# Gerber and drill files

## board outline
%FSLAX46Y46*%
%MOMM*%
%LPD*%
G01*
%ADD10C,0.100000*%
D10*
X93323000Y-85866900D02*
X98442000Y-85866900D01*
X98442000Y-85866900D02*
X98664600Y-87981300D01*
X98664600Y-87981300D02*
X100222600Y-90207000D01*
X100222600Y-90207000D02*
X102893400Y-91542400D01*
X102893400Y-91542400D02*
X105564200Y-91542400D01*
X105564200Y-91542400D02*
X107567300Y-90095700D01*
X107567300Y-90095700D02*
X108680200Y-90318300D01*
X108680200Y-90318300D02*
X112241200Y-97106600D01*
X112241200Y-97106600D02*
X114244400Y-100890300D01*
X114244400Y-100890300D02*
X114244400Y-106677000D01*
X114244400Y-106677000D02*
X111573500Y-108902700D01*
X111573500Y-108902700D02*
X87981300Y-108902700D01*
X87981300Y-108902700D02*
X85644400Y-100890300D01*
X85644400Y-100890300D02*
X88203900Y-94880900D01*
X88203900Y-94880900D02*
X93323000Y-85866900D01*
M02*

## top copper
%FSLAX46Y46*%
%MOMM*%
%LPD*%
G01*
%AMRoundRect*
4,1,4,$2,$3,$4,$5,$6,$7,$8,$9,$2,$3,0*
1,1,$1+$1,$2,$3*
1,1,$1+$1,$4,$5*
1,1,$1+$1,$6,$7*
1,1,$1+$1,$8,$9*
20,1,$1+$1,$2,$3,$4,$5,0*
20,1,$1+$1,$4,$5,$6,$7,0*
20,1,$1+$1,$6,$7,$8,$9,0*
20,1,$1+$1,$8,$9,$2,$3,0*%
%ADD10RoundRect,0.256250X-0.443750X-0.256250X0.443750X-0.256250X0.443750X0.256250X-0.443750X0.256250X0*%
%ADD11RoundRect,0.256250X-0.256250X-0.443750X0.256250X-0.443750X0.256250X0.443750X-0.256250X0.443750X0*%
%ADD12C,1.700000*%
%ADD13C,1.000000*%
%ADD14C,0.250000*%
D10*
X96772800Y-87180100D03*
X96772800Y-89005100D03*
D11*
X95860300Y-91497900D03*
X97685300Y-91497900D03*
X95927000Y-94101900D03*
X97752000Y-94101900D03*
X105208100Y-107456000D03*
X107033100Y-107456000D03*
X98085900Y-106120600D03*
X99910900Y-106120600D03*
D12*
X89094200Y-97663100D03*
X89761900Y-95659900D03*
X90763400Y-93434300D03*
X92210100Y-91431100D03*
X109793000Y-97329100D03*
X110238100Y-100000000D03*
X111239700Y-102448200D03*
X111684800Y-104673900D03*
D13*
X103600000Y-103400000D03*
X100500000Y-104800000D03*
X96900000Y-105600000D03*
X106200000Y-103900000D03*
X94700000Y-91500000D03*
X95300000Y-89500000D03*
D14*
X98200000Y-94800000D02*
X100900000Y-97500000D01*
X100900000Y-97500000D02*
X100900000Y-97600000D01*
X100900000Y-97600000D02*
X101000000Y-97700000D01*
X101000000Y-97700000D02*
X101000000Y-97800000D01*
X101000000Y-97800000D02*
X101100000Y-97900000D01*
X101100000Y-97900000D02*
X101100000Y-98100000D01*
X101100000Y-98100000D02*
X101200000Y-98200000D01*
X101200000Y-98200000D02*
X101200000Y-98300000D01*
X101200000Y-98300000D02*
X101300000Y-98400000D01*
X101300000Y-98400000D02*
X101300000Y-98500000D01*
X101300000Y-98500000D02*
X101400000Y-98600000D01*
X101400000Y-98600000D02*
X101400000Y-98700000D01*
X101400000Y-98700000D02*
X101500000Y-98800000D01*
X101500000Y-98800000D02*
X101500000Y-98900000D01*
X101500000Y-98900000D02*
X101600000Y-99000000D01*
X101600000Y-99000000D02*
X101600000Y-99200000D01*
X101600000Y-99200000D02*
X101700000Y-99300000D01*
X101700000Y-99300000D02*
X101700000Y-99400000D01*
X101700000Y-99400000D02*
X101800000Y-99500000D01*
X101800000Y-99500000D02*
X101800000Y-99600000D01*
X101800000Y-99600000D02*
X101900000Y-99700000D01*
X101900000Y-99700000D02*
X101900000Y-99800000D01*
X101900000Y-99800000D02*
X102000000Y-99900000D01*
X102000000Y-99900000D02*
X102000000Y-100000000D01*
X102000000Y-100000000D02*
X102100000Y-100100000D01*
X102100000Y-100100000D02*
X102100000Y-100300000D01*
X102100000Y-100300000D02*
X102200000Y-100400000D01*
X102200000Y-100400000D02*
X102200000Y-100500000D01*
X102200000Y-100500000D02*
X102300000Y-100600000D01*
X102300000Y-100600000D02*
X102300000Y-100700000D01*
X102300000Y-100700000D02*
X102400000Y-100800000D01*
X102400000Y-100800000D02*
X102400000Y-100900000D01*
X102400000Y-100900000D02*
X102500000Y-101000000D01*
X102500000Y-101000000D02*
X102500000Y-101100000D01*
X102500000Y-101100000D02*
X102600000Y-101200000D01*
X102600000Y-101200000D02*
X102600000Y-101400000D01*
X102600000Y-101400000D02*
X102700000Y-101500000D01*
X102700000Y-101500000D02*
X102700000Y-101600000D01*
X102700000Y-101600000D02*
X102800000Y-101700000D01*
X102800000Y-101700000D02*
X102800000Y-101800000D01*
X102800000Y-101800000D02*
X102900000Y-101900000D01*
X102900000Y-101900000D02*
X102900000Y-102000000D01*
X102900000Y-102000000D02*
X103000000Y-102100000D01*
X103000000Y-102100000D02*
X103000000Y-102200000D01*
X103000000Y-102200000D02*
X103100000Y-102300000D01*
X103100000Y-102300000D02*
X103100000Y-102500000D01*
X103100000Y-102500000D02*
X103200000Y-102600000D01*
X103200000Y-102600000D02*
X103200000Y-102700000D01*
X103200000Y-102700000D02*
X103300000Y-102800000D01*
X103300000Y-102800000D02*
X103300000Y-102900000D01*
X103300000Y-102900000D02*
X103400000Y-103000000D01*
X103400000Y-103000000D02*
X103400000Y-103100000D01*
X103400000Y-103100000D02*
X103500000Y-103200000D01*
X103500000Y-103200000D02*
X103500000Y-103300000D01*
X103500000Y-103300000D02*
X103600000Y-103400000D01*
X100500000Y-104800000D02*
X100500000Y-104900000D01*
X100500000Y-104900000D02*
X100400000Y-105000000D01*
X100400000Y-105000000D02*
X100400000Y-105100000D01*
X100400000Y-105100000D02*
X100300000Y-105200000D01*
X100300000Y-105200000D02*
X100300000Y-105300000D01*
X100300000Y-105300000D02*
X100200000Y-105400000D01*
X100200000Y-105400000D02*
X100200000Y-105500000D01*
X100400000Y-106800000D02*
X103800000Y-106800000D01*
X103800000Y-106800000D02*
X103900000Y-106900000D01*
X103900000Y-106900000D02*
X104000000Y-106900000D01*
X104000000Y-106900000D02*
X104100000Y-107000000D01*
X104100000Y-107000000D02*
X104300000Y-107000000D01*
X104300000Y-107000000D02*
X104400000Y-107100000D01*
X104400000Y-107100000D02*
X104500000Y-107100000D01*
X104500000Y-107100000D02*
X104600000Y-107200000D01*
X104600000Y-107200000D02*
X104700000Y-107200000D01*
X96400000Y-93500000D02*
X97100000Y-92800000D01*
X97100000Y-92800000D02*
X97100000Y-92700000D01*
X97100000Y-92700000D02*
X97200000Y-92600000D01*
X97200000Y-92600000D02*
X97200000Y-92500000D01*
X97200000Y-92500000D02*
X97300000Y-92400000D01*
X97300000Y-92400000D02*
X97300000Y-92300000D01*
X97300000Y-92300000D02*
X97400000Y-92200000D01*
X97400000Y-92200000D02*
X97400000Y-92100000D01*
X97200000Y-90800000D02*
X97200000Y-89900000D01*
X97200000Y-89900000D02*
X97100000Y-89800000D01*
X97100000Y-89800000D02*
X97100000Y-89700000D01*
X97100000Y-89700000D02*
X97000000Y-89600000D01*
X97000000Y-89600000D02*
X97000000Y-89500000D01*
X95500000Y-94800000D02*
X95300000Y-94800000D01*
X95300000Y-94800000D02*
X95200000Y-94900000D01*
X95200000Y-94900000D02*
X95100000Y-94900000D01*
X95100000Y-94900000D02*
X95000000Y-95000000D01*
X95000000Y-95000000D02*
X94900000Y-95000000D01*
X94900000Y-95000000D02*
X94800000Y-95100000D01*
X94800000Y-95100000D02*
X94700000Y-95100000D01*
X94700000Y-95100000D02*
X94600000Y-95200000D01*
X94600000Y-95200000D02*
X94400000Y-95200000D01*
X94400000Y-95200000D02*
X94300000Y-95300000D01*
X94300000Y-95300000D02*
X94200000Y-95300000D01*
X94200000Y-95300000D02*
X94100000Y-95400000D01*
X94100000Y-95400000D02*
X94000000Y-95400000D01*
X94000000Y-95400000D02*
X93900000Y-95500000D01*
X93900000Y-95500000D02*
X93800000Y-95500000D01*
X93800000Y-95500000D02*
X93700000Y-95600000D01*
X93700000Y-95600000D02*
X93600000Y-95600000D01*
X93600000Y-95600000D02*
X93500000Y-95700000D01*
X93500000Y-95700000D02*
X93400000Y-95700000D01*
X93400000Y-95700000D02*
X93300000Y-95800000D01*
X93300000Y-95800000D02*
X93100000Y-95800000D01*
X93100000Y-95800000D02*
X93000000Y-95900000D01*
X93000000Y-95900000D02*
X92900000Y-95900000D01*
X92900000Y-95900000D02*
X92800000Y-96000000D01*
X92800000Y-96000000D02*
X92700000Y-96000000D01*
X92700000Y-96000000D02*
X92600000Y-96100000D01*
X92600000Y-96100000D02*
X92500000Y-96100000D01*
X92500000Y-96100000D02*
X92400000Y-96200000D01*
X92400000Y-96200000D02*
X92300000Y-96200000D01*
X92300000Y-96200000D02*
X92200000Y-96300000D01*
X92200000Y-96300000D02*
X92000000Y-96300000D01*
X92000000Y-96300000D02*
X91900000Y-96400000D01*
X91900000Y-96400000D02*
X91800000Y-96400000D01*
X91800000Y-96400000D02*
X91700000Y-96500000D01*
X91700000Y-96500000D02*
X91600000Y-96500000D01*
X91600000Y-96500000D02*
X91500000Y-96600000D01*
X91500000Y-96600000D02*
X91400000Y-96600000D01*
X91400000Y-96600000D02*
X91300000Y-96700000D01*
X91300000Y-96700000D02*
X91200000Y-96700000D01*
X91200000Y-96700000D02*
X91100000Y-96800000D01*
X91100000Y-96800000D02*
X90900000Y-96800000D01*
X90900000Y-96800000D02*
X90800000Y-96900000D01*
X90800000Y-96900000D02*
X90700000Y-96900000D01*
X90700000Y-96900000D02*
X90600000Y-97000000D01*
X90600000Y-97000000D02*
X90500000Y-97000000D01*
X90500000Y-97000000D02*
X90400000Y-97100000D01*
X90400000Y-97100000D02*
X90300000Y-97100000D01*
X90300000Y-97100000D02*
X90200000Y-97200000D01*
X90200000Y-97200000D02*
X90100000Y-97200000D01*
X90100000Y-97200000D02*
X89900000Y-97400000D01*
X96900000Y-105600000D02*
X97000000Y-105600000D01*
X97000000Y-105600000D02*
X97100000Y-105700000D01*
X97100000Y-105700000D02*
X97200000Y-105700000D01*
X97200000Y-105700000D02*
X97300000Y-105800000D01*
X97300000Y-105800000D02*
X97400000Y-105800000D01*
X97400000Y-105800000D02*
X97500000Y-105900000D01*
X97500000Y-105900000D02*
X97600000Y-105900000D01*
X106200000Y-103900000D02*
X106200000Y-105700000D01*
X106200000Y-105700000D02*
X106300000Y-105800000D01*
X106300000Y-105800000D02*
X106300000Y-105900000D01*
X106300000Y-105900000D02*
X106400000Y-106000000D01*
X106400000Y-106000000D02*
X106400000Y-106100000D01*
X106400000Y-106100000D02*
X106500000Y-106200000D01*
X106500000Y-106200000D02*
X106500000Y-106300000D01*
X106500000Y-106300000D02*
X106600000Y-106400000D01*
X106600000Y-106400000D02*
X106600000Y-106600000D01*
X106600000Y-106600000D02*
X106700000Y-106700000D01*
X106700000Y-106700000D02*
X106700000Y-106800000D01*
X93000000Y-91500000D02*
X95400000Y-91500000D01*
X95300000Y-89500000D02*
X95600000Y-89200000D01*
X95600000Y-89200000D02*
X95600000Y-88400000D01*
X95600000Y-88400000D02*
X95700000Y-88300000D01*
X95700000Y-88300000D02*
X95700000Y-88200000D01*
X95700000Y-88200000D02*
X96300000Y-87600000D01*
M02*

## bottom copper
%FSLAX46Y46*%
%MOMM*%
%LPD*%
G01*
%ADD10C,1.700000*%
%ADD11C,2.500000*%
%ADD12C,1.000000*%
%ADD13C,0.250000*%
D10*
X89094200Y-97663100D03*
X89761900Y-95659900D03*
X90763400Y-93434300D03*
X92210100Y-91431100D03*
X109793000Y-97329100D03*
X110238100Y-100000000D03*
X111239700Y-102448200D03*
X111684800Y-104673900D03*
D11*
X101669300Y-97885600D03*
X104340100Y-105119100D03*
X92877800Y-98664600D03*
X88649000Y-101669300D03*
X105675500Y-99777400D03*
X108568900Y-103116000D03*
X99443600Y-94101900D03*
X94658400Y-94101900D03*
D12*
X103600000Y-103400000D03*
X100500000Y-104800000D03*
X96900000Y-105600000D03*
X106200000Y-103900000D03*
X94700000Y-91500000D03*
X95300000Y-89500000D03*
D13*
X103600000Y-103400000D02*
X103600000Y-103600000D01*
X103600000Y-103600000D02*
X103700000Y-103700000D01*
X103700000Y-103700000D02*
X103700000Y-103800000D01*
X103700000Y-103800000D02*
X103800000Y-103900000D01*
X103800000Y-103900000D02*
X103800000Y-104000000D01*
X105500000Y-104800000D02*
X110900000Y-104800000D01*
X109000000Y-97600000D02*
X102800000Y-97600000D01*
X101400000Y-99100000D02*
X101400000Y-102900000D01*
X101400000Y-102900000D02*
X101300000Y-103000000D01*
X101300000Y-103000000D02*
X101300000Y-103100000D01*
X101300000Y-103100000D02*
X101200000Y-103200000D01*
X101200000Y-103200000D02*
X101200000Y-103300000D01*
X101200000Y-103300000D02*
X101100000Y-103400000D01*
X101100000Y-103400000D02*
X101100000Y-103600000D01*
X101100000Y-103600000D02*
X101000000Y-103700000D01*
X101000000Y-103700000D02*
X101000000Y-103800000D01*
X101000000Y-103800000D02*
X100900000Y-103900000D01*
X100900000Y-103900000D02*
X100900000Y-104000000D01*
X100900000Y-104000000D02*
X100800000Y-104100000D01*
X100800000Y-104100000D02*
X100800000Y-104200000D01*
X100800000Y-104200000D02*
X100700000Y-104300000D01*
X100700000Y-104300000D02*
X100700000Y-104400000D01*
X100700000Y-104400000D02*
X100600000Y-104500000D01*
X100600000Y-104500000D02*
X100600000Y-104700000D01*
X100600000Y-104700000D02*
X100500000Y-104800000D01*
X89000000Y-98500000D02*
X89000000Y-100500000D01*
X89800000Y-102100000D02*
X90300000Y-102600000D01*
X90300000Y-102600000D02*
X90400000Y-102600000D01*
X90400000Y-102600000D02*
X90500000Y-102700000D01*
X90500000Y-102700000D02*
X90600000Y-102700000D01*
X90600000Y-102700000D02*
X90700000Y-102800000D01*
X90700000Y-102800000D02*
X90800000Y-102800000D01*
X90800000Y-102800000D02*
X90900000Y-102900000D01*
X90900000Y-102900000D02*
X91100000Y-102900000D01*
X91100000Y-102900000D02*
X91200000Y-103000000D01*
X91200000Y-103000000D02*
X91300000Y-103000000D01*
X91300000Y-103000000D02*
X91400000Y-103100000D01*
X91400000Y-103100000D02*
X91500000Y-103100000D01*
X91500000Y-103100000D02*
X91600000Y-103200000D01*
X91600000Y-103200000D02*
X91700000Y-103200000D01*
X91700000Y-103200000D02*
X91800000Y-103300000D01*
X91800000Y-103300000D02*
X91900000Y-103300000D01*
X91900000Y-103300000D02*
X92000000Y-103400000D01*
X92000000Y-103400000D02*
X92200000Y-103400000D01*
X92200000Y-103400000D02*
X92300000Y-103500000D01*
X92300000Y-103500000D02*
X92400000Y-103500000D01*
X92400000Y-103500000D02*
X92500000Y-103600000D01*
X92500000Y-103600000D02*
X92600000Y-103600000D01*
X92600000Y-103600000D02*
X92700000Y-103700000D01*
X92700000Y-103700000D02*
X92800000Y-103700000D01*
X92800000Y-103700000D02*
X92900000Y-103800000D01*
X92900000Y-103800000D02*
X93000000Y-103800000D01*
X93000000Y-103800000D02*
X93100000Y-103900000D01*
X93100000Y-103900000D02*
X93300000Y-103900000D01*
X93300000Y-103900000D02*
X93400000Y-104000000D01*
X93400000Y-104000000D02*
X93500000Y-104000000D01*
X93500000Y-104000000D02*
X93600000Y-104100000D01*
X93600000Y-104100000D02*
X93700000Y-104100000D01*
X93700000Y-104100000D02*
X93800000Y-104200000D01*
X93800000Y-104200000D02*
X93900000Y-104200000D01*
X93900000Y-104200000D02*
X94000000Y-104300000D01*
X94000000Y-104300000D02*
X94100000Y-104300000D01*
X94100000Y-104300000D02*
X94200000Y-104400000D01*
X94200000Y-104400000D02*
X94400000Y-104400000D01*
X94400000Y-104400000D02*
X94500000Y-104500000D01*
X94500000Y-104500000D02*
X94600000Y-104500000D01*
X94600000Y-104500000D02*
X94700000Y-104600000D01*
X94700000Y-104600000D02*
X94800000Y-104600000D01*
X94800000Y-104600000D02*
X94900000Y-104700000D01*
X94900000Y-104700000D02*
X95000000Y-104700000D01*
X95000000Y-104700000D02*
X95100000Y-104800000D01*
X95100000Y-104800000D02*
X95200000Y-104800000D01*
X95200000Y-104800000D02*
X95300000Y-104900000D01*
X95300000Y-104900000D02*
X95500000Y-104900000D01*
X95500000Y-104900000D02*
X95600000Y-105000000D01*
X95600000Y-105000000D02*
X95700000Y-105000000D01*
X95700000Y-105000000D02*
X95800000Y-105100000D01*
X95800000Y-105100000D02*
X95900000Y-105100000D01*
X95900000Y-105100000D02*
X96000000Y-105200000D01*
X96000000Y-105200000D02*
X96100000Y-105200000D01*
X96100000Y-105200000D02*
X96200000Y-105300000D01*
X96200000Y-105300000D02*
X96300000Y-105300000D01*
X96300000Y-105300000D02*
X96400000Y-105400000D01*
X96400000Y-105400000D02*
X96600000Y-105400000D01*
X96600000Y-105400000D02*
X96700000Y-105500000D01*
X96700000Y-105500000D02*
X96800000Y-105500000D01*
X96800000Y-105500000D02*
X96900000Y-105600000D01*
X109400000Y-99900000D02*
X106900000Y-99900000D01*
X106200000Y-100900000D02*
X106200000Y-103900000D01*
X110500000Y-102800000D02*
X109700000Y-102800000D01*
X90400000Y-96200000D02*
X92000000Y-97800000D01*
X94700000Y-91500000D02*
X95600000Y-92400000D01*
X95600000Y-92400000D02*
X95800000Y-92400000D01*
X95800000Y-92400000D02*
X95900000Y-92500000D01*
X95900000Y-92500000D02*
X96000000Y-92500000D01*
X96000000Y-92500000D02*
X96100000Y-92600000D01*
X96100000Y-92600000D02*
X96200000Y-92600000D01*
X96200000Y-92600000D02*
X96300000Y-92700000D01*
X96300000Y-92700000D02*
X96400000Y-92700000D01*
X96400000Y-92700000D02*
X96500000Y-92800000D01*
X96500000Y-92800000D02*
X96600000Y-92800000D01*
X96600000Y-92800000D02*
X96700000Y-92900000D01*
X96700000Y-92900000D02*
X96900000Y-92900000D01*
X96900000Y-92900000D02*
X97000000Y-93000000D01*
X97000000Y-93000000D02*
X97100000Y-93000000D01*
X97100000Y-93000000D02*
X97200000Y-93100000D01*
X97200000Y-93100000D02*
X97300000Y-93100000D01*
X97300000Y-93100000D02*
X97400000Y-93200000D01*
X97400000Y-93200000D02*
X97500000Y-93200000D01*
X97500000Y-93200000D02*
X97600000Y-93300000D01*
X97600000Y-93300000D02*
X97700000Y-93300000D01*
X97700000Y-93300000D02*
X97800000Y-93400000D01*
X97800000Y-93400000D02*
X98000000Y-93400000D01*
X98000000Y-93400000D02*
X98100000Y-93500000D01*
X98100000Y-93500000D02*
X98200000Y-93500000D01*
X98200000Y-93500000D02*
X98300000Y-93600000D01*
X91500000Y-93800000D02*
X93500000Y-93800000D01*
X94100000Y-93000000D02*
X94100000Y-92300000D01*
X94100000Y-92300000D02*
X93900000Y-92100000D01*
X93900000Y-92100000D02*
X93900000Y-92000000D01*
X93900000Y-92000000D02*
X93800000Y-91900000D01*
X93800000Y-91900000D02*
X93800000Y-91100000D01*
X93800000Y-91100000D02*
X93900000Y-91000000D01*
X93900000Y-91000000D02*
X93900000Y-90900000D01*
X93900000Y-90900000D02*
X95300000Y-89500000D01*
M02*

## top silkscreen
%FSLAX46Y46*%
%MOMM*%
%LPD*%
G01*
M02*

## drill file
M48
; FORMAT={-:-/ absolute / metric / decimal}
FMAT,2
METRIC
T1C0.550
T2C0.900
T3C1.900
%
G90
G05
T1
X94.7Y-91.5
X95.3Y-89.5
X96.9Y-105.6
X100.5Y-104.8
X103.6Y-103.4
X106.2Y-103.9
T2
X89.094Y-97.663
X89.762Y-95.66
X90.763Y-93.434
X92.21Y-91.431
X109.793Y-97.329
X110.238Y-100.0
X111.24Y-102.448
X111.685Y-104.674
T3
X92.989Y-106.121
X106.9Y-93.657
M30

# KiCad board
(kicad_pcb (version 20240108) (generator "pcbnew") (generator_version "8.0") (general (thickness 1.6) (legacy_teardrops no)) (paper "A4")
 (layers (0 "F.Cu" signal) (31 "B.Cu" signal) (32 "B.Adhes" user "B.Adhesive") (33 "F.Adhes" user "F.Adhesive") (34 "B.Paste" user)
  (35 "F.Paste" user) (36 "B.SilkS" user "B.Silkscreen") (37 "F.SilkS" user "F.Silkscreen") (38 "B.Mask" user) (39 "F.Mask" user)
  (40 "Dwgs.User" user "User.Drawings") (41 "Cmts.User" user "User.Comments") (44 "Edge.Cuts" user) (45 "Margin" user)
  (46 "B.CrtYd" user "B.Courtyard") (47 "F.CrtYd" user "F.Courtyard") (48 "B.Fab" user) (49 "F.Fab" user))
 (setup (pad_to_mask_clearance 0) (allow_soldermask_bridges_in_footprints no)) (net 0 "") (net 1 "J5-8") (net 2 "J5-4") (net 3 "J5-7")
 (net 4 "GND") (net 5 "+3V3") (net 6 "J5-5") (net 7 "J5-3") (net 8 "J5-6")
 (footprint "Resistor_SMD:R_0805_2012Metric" (layer "F.Cu") (at 96.7728 88.0926)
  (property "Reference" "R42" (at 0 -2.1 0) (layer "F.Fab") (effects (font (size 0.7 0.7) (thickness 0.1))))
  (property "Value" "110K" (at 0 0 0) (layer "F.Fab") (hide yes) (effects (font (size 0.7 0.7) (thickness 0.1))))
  (pad "1" smd roundrect (at 0 -0.9125) (size 1.4 1.025) (layers "F.Cu" "F.Mask" "F.Paste") (roundrect_rratio 0.25) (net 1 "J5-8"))
  (pad "2" smd roundrect (at 0 0.9125) (size 1.4 1.025) (layers "F.Cu" "F.Mask" "F.Paste") (roundrect_rratio 0.25) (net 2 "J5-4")))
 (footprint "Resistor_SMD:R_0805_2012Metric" (layer "F.Cu") (at 96.7728 91.4979)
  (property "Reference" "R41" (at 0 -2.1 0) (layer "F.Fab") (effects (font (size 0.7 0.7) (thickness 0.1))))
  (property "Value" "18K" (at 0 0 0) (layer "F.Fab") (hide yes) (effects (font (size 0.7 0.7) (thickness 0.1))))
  (pad "1" smd roundrect (at -0.9125 0) (size 1.025 1.4) (layers "F.Cu" "F.Mask" "F.Paste") (roundrect_rratio 0.25) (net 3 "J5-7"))
  (pad "2" smd roundrect (at 0.9125 0) (size 1.025 1.4) (layers "F.Cu" "F.Mask" "F.Paste") (roundrect_rratio 0.25) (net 2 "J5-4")))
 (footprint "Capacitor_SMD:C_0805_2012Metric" (layer "F.Cu") (at 96.8395 94.1019)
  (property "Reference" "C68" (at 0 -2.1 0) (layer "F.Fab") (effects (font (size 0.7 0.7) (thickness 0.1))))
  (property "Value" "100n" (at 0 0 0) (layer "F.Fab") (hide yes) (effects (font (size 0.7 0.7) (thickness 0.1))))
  (pad "1" smd roundrect (at -0.9125 0) (size 1.025 1.4) (layers "F.Cu" "F.Mask" "F.Paste") (roundrect_rratio 0.25) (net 2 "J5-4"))
  (pad "2" smd roundrect (at 0.9125 0) (size 1.025 1.4) (layers "F.Cu" "F.Mask" "F.Paste") (roundrect_rratio 0.25) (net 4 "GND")))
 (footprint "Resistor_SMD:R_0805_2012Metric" (layer "F.Cu") (at 106.1206 107.456)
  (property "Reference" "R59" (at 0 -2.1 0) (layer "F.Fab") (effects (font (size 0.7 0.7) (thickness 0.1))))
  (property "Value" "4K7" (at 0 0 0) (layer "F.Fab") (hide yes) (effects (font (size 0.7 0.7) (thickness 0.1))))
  (pad "1" smd roundrect (at -0.9125 0) (size 1.025 1.4) (layers "F.Cu" "F.Mask" "F.Paste") (roundrect_rratio 0.25) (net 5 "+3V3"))
  (pad "2" smd roundrect (at 0.9125 0) (size 1.025 1.4) (layers "F.Cu" "F.Mask" "F.Paste") (roundrect_rratio 0.25) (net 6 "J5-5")))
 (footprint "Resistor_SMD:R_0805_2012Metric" (layer "F.Cu") (at 98.9984 106.1206)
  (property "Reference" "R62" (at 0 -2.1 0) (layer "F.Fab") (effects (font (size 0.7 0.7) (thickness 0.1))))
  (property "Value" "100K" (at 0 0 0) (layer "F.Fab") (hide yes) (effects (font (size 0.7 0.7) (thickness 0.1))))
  (pad "1" smd roundrect (at -0.9125 0) (size 1.025 1.4) (layers "F.Cu" "F.Mask" "F.Paste") (roundrect_rratio 0.25) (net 2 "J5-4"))
  (pad "2" smd roundrect (at 0.9125 0) (size 1.025 1.4) (layers "F.Cu" "F.Mask" "F.Paste") (roundrect_rratio 0.25) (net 5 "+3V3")))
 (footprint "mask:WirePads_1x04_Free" (layer "F.Cu") (at 90.4574 94.5471)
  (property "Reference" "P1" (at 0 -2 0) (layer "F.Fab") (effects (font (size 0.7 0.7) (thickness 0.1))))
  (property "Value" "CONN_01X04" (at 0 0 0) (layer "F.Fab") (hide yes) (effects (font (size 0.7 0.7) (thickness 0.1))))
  (pad "1" thru_hole circle (at -1.3632 3.116) (size 1.7 1.7) (drill 0.9) (layers "*.Cu" "*.Mask") (remove_unused_layers no) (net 2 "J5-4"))
  (pad "2" thru_hole circle (at -0.6955 1.1128) (size 1.7 1.7) (drill 0.9) (layers "*.Cu" "*.Mask") (remove_unused_layers no) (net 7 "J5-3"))
  (pad "3" thru_hole circle (at 0.306 -1.1128) (size 1.7 1.7) (drill 0.9) (layers "*.Cu" "*.Mask") (remove_unused_layers no) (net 1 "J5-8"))
  (pad "4" thru_hole circle (at 1.7527 -3.116) (size 1.7 1.7) (drill 0.9) (layers "*.Cu" "*.Mask") (remove_unused_layers no) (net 3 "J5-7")))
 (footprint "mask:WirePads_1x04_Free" (layer "F.Cu") (at 110.7389 101.1128)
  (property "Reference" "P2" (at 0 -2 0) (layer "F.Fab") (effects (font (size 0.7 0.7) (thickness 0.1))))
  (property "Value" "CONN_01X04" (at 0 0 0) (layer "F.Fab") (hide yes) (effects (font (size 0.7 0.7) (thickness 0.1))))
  (pad "1" thru_hole circle (at -0.9459 -3.7837) (size 1.7 1.7) (drill 0.9) (layers "*.Cu" "*.Mask") (remove_unused_layers no)
   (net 5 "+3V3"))
  (pad "2" thru_hole circle (at -0.5008 -1.1128) (size 1.7 1.7) (drill 0.9) (layers "*.Cu" "*.Mask") (remove_unused_layers no)
   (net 6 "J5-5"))
  (pad "3" thru_hole circle (at 0.5008 1.3354) (size 1.7 1.7) (drill 0.9) (layers "*.Cu" "*.Mask") (remove_unused_layers no) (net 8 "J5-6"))
  (pad "4" thru_hole circle (at 0.9459 3.5611) (size 1.7 1.7) (drill 0.9) (layers "*.Cu" "*.Mask") (remove_unused_layers no) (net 4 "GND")))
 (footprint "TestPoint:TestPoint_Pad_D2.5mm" (layer "B.Cu") (at 101.6693 97.8856)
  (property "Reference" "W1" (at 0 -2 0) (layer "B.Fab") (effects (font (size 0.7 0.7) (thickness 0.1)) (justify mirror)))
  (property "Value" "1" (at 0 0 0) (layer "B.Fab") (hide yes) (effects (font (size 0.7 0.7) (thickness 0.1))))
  (pad "1" smd circle (at 0 0) (size 2.5 2.5) (layers "B.Cu" "B.Mask") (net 5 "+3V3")))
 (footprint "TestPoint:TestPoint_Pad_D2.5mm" (layer "B.Cu") (at 104.3401 105.1191)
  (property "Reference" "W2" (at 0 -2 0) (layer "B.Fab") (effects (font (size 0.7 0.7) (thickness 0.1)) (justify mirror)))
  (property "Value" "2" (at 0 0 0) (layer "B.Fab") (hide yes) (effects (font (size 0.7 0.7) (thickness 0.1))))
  (pad "1" smd circle (at 0 0) (size 2.5 2.5) (layers "B.Cu" "B.Mask") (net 4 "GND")))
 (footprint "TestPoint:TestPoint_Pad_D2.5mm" (layer "B.Cu") (at 92.8778 98.6646)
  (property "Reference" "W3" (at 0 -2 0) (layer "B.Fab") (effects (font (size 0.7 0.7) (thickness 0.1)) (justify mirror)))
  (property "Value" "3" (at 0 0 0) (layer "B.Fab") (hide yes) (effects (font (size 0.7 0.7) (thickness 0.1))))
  (pad "1" smd circle (at 0 0) (size 2.5 2.5) (layers "B.Cu" "B.Mask") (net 7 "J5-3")))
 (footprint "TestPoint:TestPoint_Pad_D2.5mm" (layer "B.Cu") (at 88.649 101.6693)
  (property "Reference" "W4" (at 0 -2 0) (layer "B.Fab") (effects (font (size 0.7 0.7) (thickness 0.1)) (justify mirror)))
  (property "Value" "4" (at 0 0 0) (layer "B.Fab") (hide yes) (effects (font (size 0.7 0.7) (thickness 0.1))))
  (pad "1" smd circle (at 0 0) (size 2.5 2.5) (layers "B.Cu" "B.Mask") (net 2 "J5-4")))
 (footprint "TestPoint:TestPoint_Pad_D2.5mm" (layer "B.Cu") (at 105.6755 99.7774)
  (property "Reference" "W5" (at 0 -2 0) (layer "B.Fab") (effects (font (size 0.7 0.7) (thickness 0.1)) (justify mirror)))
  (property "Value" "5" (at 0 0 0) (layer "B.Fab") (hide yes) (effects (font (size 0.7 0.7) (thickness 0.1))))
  (pad "1" smd circle (at 0 0) (size 2.5 2.5) (layers "B.Cu" "B.Mask") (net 6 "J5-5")))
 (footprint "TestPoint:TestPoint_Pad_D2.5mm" (layer "B.Cu") (at 108.5689 103.116)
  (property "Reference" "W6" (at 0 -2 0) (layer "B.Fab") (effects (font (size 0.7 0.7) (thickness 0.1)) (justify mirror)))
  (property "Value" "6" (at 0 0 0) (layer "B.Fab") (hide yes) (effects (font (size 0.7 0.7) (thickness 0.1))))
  (pad "1" smd circle (at 0 0) (size 2.5 2.5) (layers "B.Cu" "B.Mask") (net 8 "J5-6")))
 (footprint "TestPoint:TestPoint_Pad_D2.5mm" (layer "B.Cu") (at 99.4436 94.1019)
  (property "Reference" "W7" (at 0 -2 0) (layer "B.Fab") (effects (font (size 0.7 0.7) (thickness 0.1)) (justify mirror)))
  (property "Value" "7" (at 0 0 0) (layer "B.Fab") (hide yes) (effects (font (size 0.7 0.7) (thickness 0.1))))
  (pad "1" smd circle (at 0 0) (size 2.5 2.5) (layers "B.Cu" "B.Mask") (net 3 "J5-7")))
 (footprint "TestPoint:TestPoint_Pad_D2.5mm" (layer "B.Cu") (at 94.6584 94.1019)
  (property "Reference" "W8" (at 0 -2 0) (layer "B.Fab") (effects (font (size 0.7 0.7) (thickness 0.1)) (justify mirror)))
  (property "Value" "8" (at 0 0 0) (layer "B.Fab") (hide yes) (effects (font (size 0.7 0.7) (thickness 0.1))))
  (pad "1" smd circle (at 0 0) (size 2.5 2.5) (layers "B.Cu" "B.Mask") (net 1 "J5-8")))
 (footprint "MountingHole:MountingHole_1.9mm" (layer "F.Cu") (at 92.9891 106.1206)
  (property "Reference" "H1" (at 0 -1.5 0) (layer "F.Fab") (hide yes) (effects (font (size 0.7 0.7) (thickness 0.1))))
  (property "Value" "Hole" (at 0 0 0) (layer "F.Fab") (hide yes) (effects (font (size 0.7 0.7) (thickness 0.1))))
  (pad "" np_thru_hole circle (at 0 0) (size 1.9 1.9) (drill 1.9) (layers "*.Cu" "*.Mask")))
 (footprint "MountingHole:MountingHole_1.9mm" (layer "F.Cu") (at 106.8996 93.6568)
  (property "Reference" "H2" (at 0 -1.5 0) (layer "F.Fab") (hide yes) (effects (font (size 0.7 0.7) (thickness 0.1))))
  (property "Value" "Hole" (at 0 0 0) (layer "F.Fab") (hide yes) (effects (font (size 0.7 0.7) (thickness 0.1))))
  (pad "" np_thru_hole circle (at 0 0) (size 1.9 1.9) (drill 1.9) (layers "*.Cu" "*.Mask")))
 (segment (start 98.2 94.8) (end 100.9 97.5) (width 0.25) (layer "F.Cu") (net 4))
 (segment (start 100.9 97.5) (end 100.9 97.6) (width 0.25) (layer "F.Cu") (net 4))
 (segment (start 100.9 97.6) (end 101 97.7) (width 0.25) (layer "F.Cu") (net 4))
 (segment (start 101 97.7) (end 101 97.8) (width 0.25) (layer "F.Cu") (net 4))
 (segment (start 101 97.8) (end 101.1 97.9) (width 0.25) (layer "F.Cu") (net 4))
 (segment (start 101.1 97.9) (end 101.1 98.1) (width 0.25) (layer "F.Cu") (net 4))
 (segment (start 101.1 98.1) (end 101.2 98.2) (width 0.25) (layer "F.Cu") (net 4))
 (segment (start 101.2 98.2) (end 101.2 98.3) (width 0.25) (layer "F.Cu") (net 4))
 (segment (start 101.2 98.3) (end 101.3 98.4) (width 0.25) (layer "F.Cu") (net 4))
 (segment (start 101.3 98.4) (end 101.3 98.5) (width 0.25) (layer "F.Cu") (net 4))
 (segment (start 101.3 98.5) (end 101.4 98.6) (width 0.25) (layer "F.Cu") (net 4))
 (segment (start 101.4 98.6) (end 101.4 98.7) (width 0.25) (layer "F.Cu") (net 4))
 (segment (start 101.4 98.7) (end 101.5 98.8) (width 0.25) (layer "F.Cu") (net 4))
 (segment (start 101.5 98.8) (end 101.5 98.9) (width 0.25) (layer "F.Cu") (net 4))
 (segment (start 101.5 98.9) (end 101.6 99) (width 0.25) (layer "F.Cu") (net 4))
 (segment (start 101.6 99) (end 101.6 99.2) (width 0.25) (layer "F.Cu") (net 4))
 (segment (start 101.6 99.2) (end 101.7 99.3) (width 0.25) (layer "F.Cu") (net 4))
 (segment (start 101.7 99.3) (end 101.7 99.4) (width 0.25) (layer "F.Cu") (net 4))
 (segment (start 101.7 99.4) (end 101.8 99.5) (width 0.25) (layer "F.Cu") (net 4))
 (segment (start 101.8 99.5) (end 101.8 99.6) (width 0.25) (layer "F.Cu") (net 4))
 (segment (start 101.8 99.6) (end 101.9 99.7) (width 0.25) (layer "F.Cu") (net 4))
 (segment (start 101.9 99.7) (end 101.9 99.8) (width 0.25) (layer "F.Cu") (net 4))
 (segment (start 101.9 99.8) (end 102 99.9) (width 0.25) (layer "F.Cu") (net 4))
 (segment (start 102 99.9) (end 102 100) (width 0.25) (layer "F.Cu") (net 4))
 (segment (start 102 100) (end 102.1 100.1) (width 0.25) (layer "F.Cu") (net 4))
 (segment (start 102.1 100.1) (end 102.1 100.3) (width 0.25) (layer "F.Cu") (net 4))
 (segment (start 102.1 100.3) (end 102.2 100.4) (width 0.25) (layer "F.Cu") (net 4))
 (segment (start 102.2 100.4) (end 102.2 100.5) (width 0.25) (layer "F.Cu") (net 4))
 (segment (start 102.2 100.5) (end 102.3 100.6) (width 0.25) (layer "F.Cu") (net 4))
 (segment (start 102.3 100.6) (end 102.3 100.7) (width 0.25) (layer "F.Cu") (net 4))
 (segment (start 102.3 100.7) (end 102.4 100.8) (width 0.25) (layer "F.Cu") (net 4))
 (segment (start 102.4 100.8) (end 102.4 100.9) (width 0.25) (layer "F.Cu") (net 4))
 (segment (start 102.4 100.9) (end 102.5 101) (width 0.25) (layer "F.Cu") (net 4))
 (segment (start 102.5 101) (end 102.5 101.1) (width 0.25) (layer "F.Cu") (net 4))
 (segment (start 102.5 101.1) (end 102.6 101.2) (width 0.25) (layer "F.Cu") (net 4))
 (segment (start 102.6 101.2) (end 102.6 101.4) (width 0.25) (layer "F.Cu") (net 4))
 (segment (start 102.6 101.4) (end 102.7 101.5) (width 0.25) (layer "F.Cu") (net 4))
 (segment (start 102.7 101.5) (end 102.7 101.6) (width 0.25) (layer "F.Cu") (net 4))
 (segment (start 102.7 101.6) (end 102.8 101.7) (width 0.25) (layer "F.Cu") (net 4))
 (segment (start 102.8 101.7) (end 102.8 101.8) (width 0.25) (layer "F.Cu") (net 4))
 (segment (start 102.8 101.8) (end 102.9 101.9) (width 0.25) (layer "F.Cu") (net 4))
 (segment (start 102.9 101.9) (end 102.9 102) (width 0.25) (layer "F.Cu") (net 4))
 (segment (start 102.9 102) (end 103 102.1) (width 0.25) (layer "F.Cu") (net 4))
 (segment (start 103 102.1) (end 103 102.2) (width 0.25) (layer "F.Cu") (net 4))
 (segment (start 103 102.2) (end 103.1 102.3) (width 0.25) (layer "F.Cu") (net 4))
 (segment (start 103.1 102.3) (end 103.1 102.5) (width 0.25) (layer "F.Cu") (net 4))
 (segment (start 103.1 102.5) (end 103.2 102.6) (width 0.25) (layer "F.Cu") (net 4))
 (segment (start 103.2 102.6) (end 103.2 102.7) (width 0.25) (layer "F.Cu") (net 4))
 (segment (start 103.2 102.7) (end 103.3 102.8) (width 0.25) (layer "F.Cu") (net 4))
 (segment (start 103.3 102.8) (end 103.3 102.9) (width 0.25) (layer "F.Cu") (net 4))
 (segment (start 103.3 102.9) (end 103.4 103) (width 0.25) (layer "F.Cu") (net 4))
 (segment (start 103.4 103) (end 103.4 103.1) (width 0.25) (layer "F.Cu") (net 4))
 (segment (start 103.4 103.1) (end 103.5 103.2) (width 0.25) (layer "F.Cu") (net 4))
 (segment (start 103.5 103.2) (end 103.5 103.3) (width 0.25) (layer "F.Cu") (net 4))
 (segment (start 103.5 103.3) (end 103.6 103.4) (width 0.25) (layer "F.Cu") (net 4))
 (segment (start 103.6 103.4) (end 103.6 103.6) (width 0.25) (layer "B.Cu") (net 4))
 (segment (start 103.6 103.6) (end 103.7 103.7) (width 0.25) (layer "B.Cu") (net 4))
 (segment (start 103.7 103.7) (end 103.7 103.8) (width 0.25) (layer "B.Cu") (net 4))
 (segment (start 103.7 103.8) (end 103.8 103.9) (width 0.25) (layer "B.Cu") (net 4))
 (segment (start 103.8 103.9) (end 103.8 104) (width 0.25) (layer "B.Cu") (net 4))
 (segment (start 105.5 104.8) (end 110.9 104.8) (width 0.25) (layer "B.Cu") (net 4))
 (via (at 103.6 103.4) (size 1) (drill 0.55) (layers "F.Cu" "B.Cu") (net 4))
 (segment (start 109 97.6) (end 102.8 97.6) (width 0.25) (layer "B.Cu") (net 5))
 (segment (start 101.4 99.1) (end 101.4 102.9) (width 0.25) (layer "B.Cu") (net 5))
 (segment (start 101.4 102.9) (end 101.3 103) (width 0.25) (layer "B.Cu") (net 5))
 (segment (start 101.3 103) (end 101.3 103.1) (width 0.25) (layer "B.Cu") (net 5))
 (segment (start 101.3 103.1) (end 101.2 103.2) (width 0.25) (layer "B.Cu") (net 5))
 (segment (start 101.2 103.2) (end 101.2 103.3) (width 0.25) (layer "B.Cu") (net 5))
 (segment (start 101.2 103.3) (end 101.1 103.4) (width 0.25) (layer "B.Cu") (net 5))
 (segment (start 101.1 103.4) (end 101.1 103.6) (width 0.25) (layer "B.Cu") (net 5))
 (segment (start 101.1 103.6) (end 101 103.7) (width 0.25) (layer "B.Cu") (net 5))
 (segment (start 101 103.7) (end 101 103.8) (width 0.25) (layer "B.Cu") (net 5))
 (segment (start 101 103.8) (end 100.9 103.9) (width 0.25) (layer "B.Cu") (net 5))
 (segment (start 100.9 103.9) (end 100.9 104) (width 0.25) (layer "B.Cu") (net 5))
 (segment (start 100.9 104) (end 100.8 104.1) (width 0.25) (layer "B.Cu") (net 5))
 (segment (start 100.8 104.1) (end 100.8 104.2) (width 0.25) (layer "B.Cu") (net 5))
 (segment (start 100.8 104.2) (end 100.7 104.3) (width 0.25) (layer "B.Cu") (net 5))
 (segment (start 100.7 104.3) (end 100.7 104.4) (width 0.25) (layer "B.Cu") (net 5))
 (segment (start 100.7 104.4) (end 100.6 104.5) (width 0.25) (layer "B.Cu") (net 5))
 (segment (start 100.6 104.5) (end 100.6 104.7) (width 0.25) (layer "B.Cu") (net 5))
 (segment (start 100.6 104.7) (end 100.5 104.8) (width 0.25) (layer "B.Cu") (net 5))
 (segment (start 100.5 104.8) (end 100.5 104.9) (width 0.25) (layer "F.Cu") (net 5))
 (segment (start 100.5 104.9) (end 100.4 105) (width 0.25) (layer "F.Cu") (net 5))
 (segment (start 100.4 105) (end 100.4 105.1) (width 0.25) (layer "F.Cu") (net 5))
 (segment (start 100.4 105.1) (end 100.3 105.2) (width 0.25) (layer "F.Cu") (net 5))
 (segment (start 100.3 105.2) (end 100.3 105.3) (width 0.25) (layer "F.Cu") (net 5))
 (segment (start 100.3 105.3) (end 100.2 105.4) (width 0.25) (layer "F.Cu") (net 5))
 (segment (start 100.2 105.4) (end 100.2 105.5) (width 0.25) (layer "F.Cu") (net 5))
 (segment (start 100.4 106.8) (end 103.8 106.8) (width 0.25) (layer "F.Cu") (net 5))
 (segment (start 103.8 106.8) (end 103.9 106.9) (width 0.25) (layer "F.Cu") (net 5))
 (segment (start 103.9 106.9) (end 104 106.9) (width 0.25) (layer "F.Cu") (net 5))
 (segment (start 104 106.9) (end 104.1 107) (width 0.25) (layer "F.Cu") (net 5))
 (segment (start 104.1 107) (end 104.3 107) (width 0.25) (layer "F.Cu") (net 5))
 (segment (start 104.3 107) (end 104.4 107.1) (width 0.25) (layer "F.Cu") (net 5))
 (segment (start 104.4 107.1) (end 104.5 107.1) (width 0.25) (layer "F.Cu") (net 5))
 (segment (start 104.5 107.1) (end 104.6 107.2) (width 0.25) (layer "F.Cu") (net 5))
 (segment (start 104.6 107.2) (end 104.7 107.2) (width 0.25) (layer "F.Cu") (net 5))
 (via (at 100.5 104.8) (size 1) (drill 0.55) (layers "F.Cu" "B.Cu") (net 5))
 (segment (start 96.4 93.5) (end 97.1 92.8) (width 0.25) (layer "F.Cu") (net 2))
 (segment (start 97.1 92.8) (end 97.1 92.7) (width 0.25) (layer "F.Cu") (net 2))
 (segment (start 97.1 92.7) (end 97.2 92.6) (width 0.25) (layer "F.Cu") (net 2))
 (segment (start 97.2 92.6) (end 97.2 92.5) (width 0.25) (layer "F.Cu") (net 2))
 (segment (start 97.2 92.5) (end 97.3 92.4) (width 0.25) (layer "F.Cu") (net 2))
 (segment (start 97.3 92.4) (end 97.3 92.3) (width 0.25) (layer "F.Cu") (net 2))
 (segment (start 97.3 92.3) (end 97.4 92.2) (width 0.25) (layer "F.Cu") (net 2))
 (segment (start 97.4 92.2) (end 97.4 92.1) (width 0.25) (layer "F.Cu") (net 2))
 (segment (start 97.2 90.8) (end 97.2 89.9) (width 0.25) (layer "F.Cu") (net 2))
 (segment (start 97.2 89.9) (end 97.1 89.8) (width 0.25) (layer "F.Cu") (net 2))
 (segment (start 97.1 89.8) (end 97.1 89.7) (width 0.25) (layer "F.Cu") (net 2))
 (segment (start 97.1 89.7) (end 97 89.6) (width 0.25) (layer "F.Cu") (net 2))
 (segment (start 97 89.6) (end 97 89.5) (width 0.25) (layer "F.Cu") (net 2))
 (segment (start 95.5 94.8) (end 95.3 94.8) (width 0.25) (layer "F.Cu") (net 2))
 (segment (start 95.3 94.8) (end 95.2 94.9) (width 0.25) (layer "F.Cu") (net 2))
 (segment (start 95.2 94.9) (end 95.1 94.9) (width 0.25) (layer "F.Cu") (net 2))
 (segment (start 95.1 94.9) (end 95 95) (width 0.25) (layer "F.Cu") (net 2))
 (segment (start 95 95) (end 94.9 95) (width 0.25) (layer "F.Cu") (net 2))
 (segment (start 94.9 95) (end 94.8 95.1) (width 0.25) (layer "F.Cu") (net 2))
 (segment (start 94.8 95.1) (end 94.7 95.1) (width 0.25) (layer "F.Cu") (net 2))
 (segment (start 94.7 95.1) (end 94.6 95.2) (width 0.25) (layer "F.Cu") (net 2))
 (segment (start 94.6 95.2) (end 94.4 95.2) (width 0.25) (layer "F.Cu") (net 2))
 (segment (start 94.4 95.2) (end 94.3 95.3) (width 0.25) (layer "F.Cu") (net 2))
 (segment (start 94.3 95.3) (end 94.2 95.3) (width 0.25) (layer "F.Cu") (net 2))
 (segment (start 94.2 95.3) (end 94.1 95.4) (width 0.25) (layer "F.Cu") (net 2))
 (segment (start 94.1 95.4) (end 94 95.4) (width 0.25) (layer "F.Cu") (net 2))
 (segment (start 94 95.4) (end 93.9 95.5) (width 0.25) (layer "F.Cu") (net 2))
 (segment (start 93.9 95.5) (end 93.8 95.5) (width 0.25) (layer "F.Cu") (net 2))
 (segment (start 93.8 95.5) (end 93.7 95.6) (width 0.25) (layer "F.Cu") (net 2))
 (segment (start 93.7 95.6) (end 93.6 95.6) (width 0.25) (layer "F.Cu") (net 2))
 (segment (start 93.6 95.6) (end 93.5 95.7) (width 0.25) (layer "F.Cu") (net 2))
 (segment (start 93.5 95.7) (end 93.4 95.7) (width 0.25) (layer "F.Cu") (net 2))
 (segment (start 93.4 95.7) (end 93.3 95.8) (width 0.25) (layer "F.Cu") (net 2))
 (segment (start 93.3 95.8) (end 93.1 95.8) (width 0.25) (layer "F.Cu") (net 2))
 (segment (start 93.1 95.8) (end 93 95.9) (width 0.25) (layer "F.Cu") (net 2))
 (segment (start 93 95.9) (end 92.9 95.9) (width 0.25) (layer "F.Cu") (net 2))
 (segment (start 92.9 95.9) (end 92.8 96) (width 0.25) (layer "F.Cu") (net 2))
 (segment (start 92.8 96) (end 92.7 96) (width 0.25) (layer "F.Cu") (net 2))
 (segment (start 92.7 96) (end 92.6 96.1) (width 0.25) (layer "F.Cu") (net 2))
 (segment (start 92.6 96.1) (end 92.5 96.1) (width 0.25) (layer "F.Cu") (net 2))
 (segment (start 92.5 96.1) (end 92.4 96.2) (width 0.25) (layer "F.Cu") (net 2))
 (segment (start 92.4 96.2) (end 92.3 96.2) (width 0.25) (layer "F.Cu") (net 2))
 (segment (start 92.3 96.2) (end 92.2 96.3) (width 0.25) (layer "F.Cu") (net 2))
 (segment (start 92.2 96.3) (end 92 96.3) (width 0.25) (layer "F.Cu") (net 2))
 (segment (start 92 96.3) (end 91.9 96.4) (width 0.25) (layer "F.Cu") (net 2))
 (segment (start 91.9 96.4) (end 91.8 96.4) (width 0.25) (layer "F.Cu") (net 2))
 (segment (start 91.8 96.4) (end 91.7 96.5) (width 0.25) (layer "F.Cu") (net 2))
 (segment (start 91.7 96.5) (end 91.6 96.5) (width 0.25) (layer "F.Cu") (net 2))
 (segment (start 91.6 96.5) (end 91.5 96.6) (width 0.25) (layer "F.Cu") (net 2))
 (segment (start 91.5 96.6) (end 91.4 96.6) (width 0.25) (layer "F.Cu") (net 2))
 (segment (start 91.4 96.6) (end 91.3 96.7) (width 0.25) (layer "F.Cu") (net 2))
 (segment (start 91.3 96.7) (end 91.2 96.7) (width 0.25) (layer "F.Cu") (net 2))
 (segment (start 91.2 96.7) (end 91.1 96.8) (width 0.25) (layer "F.Cu") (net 2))
 (segment (start 91.1 96.8) (end 90.9 96.8) (width 0.25) (layer "F.Cu") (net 2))
 (segment (start 90.9 96.8) (end 90.8 96.9) (width 0.25) (layer "F.Cu") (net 2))
 (segment (start 90.8 96.9) (end 90.7 96.9) (width 0.25) (layer "F.Cu") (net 2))
 (segment (start 90.7 96.9) (end 90.6 97) (width 0.25) (layer "F.Cu") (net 2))
 (segment (start 90.6 97) (end 90.5 97) (width 0.25) (layer "F.Cu") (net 2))
 (segment (start 90.5 97) (end 90.4 97.1) (width 0.25) (layer "F.Cu") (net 2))
 (segment (start 90.4 97.1) (end 90.3 97.1) (width 0.25) (layer "F.Cu") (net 2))
 (segment (start 90.3 97.1) (end 90.2 97.2) (width 0.25) (layer "F.Cu") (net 2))
 (segment (start 90.2 97.2) (end 90.1 97.2) (width 0.25) (layer "F.Cu") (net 2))
 (segment (start 90.1 97.2) (end 89.9 97.4) (width 0.25) (layer "F.Cu") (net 2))
 (segment (start 89 98.5) (end 89 100.5) (width 0.25) (layer "B.Cu") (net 2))
 (segment (start 89.8 102.1) (end 90.3 102.6) (width 0.25) (layer "B.Cu") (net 2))
 (segment (start 90.3 102.6) (end 90.4 102.6) (width 0.25) (layer "B.Cu") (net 2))
 (segment (start 90.4 102.6) (end 90.5 102.7) (width 0.25) (layer "B.Cu") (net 2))
 (segment (start 90.5 102.7) (end 90.6 102.7) (width 0.25) (layer "B.Cu") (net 2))
 (segment (start 90.6 102.7) (end 90.7 102.8) (width 0.25) (layer "B.Cu") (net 2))
 (segment (start 90.7 102.8) (end 90.8 102.8) (width 0.25) (layer "B.Cu") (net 2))
 (segment (start 90.8 102.8) (end 90.9 102.9) (width 0.25) (layer "B.Cu") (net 2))
 (segment (start 90.9 102.9) (end 91.1 102.9) (width 0.25) (layer "B.Cu") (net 2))
 (segment (start 91.1 102.9) (end 91.2 103) (width 0.25) (layer "B.Cu") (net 2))
 (segment (start 91.2 103) (end 91.3 103) (width 0.25) (layer "B.Cu") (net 2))
 (segment (start 91.3 103) (end 91.4 103.1) (width 0.25) (layer "B.Cu") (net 2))
 (segment (start 91.4 103.1) (end 91.5 103.1) (width 0.25) (layer "B.Cu") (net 2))
 (segment (start 91.5 103.1) (end 91.6 103.2) (width 0.25) (layer "B.Cu") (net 2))
 (segment (start 91.6 103.2) (end 91.7 103.2) (width 0.25) (layer "B.Cu") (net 2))
 (segment (start 91.7 103.2) (end 91.8 103.3) (width 0.25) (layer "B.Cu") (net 2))
 (segment (start 91.8 103.3) (end 91.9 103.3) (width 0.25) (layer "B.Cu") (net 2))
 (segment (start 91.9 103.3) (end 92 103.4) (width 0.25) (layer "B.Cu") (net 2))
 (segment (start 92 103.4) (end 92.2 103.4) (width 0.25) (layer "B.Cu") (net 2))
 (segment (start 92.2 103.4) (end 92.3 103.5) (width 0.25) (layer "B.Cu") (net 2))
 (segment (start 92.3 103.5) (end 92.4 103.5) (width 0.25) (layer "B.Cu") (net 2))
 (segment (start 92.4 103.5) (end 92.5 103.6) (width 0.25) (layer "B.Cu") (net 2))
 (segment (start 92.5 103.6) (end 92.6 103.6) (width 0.25) (layer "B.Cu") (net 2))
 (segment (start 92.6 103.6) (end 92.7 103.7) (width 0.25) (layer "B.Cu") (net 2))
 (segment (start 92.7 103.7) (end 92.8 103.7) (width 0.25) (layer "B.Cu") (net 2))
 (segment (start 92.8 103.7) (end 92.9 103.8) (width 0.25) (layer "B.Cu") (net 2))
 (segment (start 92.9 103.8) (end 93 103.8) (width 0.25) (layer "B.Cu") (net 2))
 (segment (start 93 103.8) (end 93.1 103.9) (width 0.25) (layer "B.Cu") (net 2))
 (segment (start 93.1 103.9) (end 93.3 103.9) (width 0.25) (layer "B.Cu") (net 2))
 (segment (start 93.3 103.9) (end 93.4 104) (width 0.25) (layer "B.Cu") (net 2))
 (segment (start 93.4 104) (end 93.5 104) (width 0.25) (layer "B.Cu") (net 2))
 (segment (start 93.5 104) (end 93.6 104.1) (width 0.25) (layer "B.Cu") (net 2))
 (segment (start 93.6 104.1) (end 93.7 104.1) (width 0.25) (layer "B.Cu") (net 2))
 (segment (start 93.7 104.1) (end 93.8 104.2) (width 0.25) (layer "B.Cu") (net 2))
 (segment (start 93.8 104.2) (end 93.9 104.2) (width 0.25) (layer "B.Cu") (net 2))
 (segment (start 93.9 104.2) (end 94 104.3) (width 0.25) (layer "B.Cu") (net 2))
 (segment (start 94 104.3) (end 94.1 104.3) (width 0.25) (layer "B.Cu") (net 2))
 (segment (start 94.1 104.3) (end 94.2 104.4) (width 0.25) (layer "B.Cu") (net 2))
 (segment (start 94.2 104.4) (end 94.4 104.4) (width 0.25) (layer "B.Cu") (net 2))
 (segment (start 94.4 104.4) (end 94.5 104.5) (width 0.25) (layer "B.Cu") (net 2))
 (segment (start 94.5 104.5) (end 94.6 104.5) (width 0.25) (layer "B.Cu") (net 2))
 (segment (start 94.6 104.5) (end 94.7 104.6) (width 0.25) (layer "B.Cu") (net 2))
 (segment (start 94.7 104.6) (end 94.8 104.6) (width 0.25) (layer "B.Cu") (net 2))
 (segment (start 94.8 104.6) (end 94.9 104.7) (width 0.25) (layer "B.Cu") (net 2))
 (segment (start 94.9 104.7) (end 95 104.7) (width 0.25) (layer "B.Cu") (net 2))
 (segment (start 95 104.7) (end 95.1 104.8) (width 0.25) (layer "B.Cu") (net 2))
 (segment (start 95.1 104.8) (end 95.2 104.8) (width 0.25) (layer "B.Cu") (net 2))
 (segment (start 95.2 104.8) (end 95.3 104.9) (width 0.25) (layer "B.Cu") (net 2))
 (segment (start 95.3 104.9) (end 95.5 104.9) (width 0.25) (layer "B.Cu") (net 2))
 (segment (start 95.5 104.9) (end 95.6 105) (width 0.25) (layer "B.Cu") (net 2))
 (segment (start 95.6 105) (end 95.7 105) (width 0.25) (layer "B.Cu") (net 2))
 (segment (start 95.7 105) (end 95.8 105.1) (width 0.25) (layer "B.Cu") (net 2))
 (segment (start 95.8 105.1) (end 95.9 105.1) (width 0.25) (layer "B.Cu") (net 2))
 (segment (start 95.9 105.1) (end 96 105.2) (width 0.25) (layer "B.Cu") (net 2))
 (segment (start 96 105.2) (end 96.1 105.2) (width 0.25) (layer "B.Cu") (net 2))
 (segment (start 96.1 105.2) (end 96.2 105.3) (width 0.25) (layer "B.Cu") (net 2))
 (segment (start 96.2 105.3) (end 96.3 105.3) (width 0.25) (layer "B.Cu") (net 2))
 (segment (start 96.3 105.3) (end 96.4 105.4) (width 0.25) (layer "B.Cu") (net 2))
 (segment (start 96.4 105.4) (end 96.6 105.4) (width 0.25) (layer "B.Cu") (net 2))
 (segment (start 96.6 105.4) (end 96.7 105.5) (width 0.25) (layer "B.Cu") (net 2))
 (segment (start 96.7 105.5) (end 96.8 105.5) (width 0.25) (layer "B.Cu") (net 2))
 (segment (start 96.8 105.5) (end 96.9 105.6) (width 0.25) (layer "B.Cu") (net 2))
 (segment (start 96.9 105.6) (end 97 105.6) (width 0.25) (layer "F.Cu") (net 2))
 (segment (start 97 105.6) (end 97.1 105.7) (width 0.25) (layer "F.Cu") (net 2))
 (segment (start 97.1 105.7) (end 97.2 105.7) (width 0.25) (layer "F.Cu") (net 2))
 (segment (start 97.2 105.7) (end 97.3 105.8) (width 0.25) (layer "F.Cu") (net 2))
 (segment (start 97.3 105.8) (end 97.4 105.8) (width 0.25) (layer "F.Cu") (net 2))
 (segment (start 97.4 105.8) (end 97.5 105.9) (width 0.25) (layer "F.Cu") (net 2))
 (segment (start 97.5 105.9) (end 97.6 105.9) (width 0.25) (layer "F.Cu") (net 2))
 (via (at 96.9 105.6) (size 1) (drill 0.55) (layers "F.Cu" "B.Cu") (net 2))
 (segment (start 109.4 99.9) (end 106.9 99.9) (width 0.25) (layer "B.Cu") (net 6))
 (segment (start 106.2 100.9) (end 106.2 103.9) (width 0.25) (layer "B.Cu") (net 6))
 (segment (start 106.2 103.9) (end 106.2 105.7) (width 0.25) (layer "F.Cu") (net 6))
 (segment (start 106.2 105.7) (end 106.3 105.8) (width 0.25) (layer "F.Cu") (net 6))
 (segment (start 106.3 105.8) (end 106.3 105.9) (width 0.25) (layer "F.Cu") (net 6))
 (segment (start 106.3 105.9) (end 106.4 106) (width 0.25) (layer "F.Cu") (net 6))
 (segment (start 106.4 106) (end 106.4 106.1) (width 0.25) (layer "F.Cu") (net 6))
 (segment (start 106.4 106.1) (end 106.5 106.2) (width 0.25) (layer "F.Cu") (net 6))
 (segment (start 106.5 106.2) (end 106.5 106.3) (width 0.25) (layer "F.Cu") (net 6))
 (segment (start 106.5 106.3) (end 106.6 106.4) (width 0.25) (layer "F.Cu") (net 6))
 (segment (start 106.6 106.4) (end 106.6 106.6) (width 0.25) (layer "F.Cu") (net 6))
 (segment (start 106.6 106.6) (end 106.7 106.7) (width 0.25) (layer "F.Cu") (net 6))
 (segment (start 106.7 106.7) (end 106.7 106.8) (width 0.25) (layer "F.Cu") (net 6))
 (via (at 106.2 103.9) (size 1) (drill 0.55) (layers "F.Cu" "B.Cu") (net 6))
 (segment (start 110.5 102.8) (end 109.7 102.8) (width 0.25) (layer "B.Cu") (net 8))
 (segment (start 90.4 96.2) (end 92 97.8) (width 0.25) (layer "B.Cu") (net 7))
 (segment (start 93 91.5) (end 95.4 91.5) (width 0.25) (layer "F.Cu") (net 3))
 (segment (start 94.7 91.5) (end 95.6 92.4) (width 0.25) (layer "B.Cu") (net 3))
 (segment (start 95.6 92.4) (end 95.8 92.4) (width 0.25) (layer "B.Cu") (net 3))
 (segment (start 95.8 92.4) (end 95.9 92.5) (width 0.25) (layer "B.Cu") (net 3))
 (segment (start 95.9 92.5) (end 96 92.5) (width 0.25) (layer "B.Cu") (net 3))
 (segment (start 96 92.5) (end 96.1 92.6) (width 0.25) (layer "B.Cu") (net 3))
 (segment (start 96.1 92.6) (end 96.2 92.6) (width 0.25) (layer "B.Cu") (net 3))
 (segment (start 96.2 92.6) (end 96.3 92.7) (width 0.25) (layer "B.Cu") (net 3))
 (segment (start 96.3 92.7) (end 96.4 92.7) (width 0.25) (layer "B.Cu") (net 3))
 (segment (start 96.4 92.7) (end 96.5 92.8) (width 0.25) (layer "B.Cu") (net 3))
 (segment (start 96.5 92.8) (end 96.6 92.8) (width 0.25) (layer "B.Cu") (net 3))
 (segment (start 96.6 92.8) (end 96.7 92.9) (width 0.25) (layer "B.Cu") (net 3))
 (segment (start 96.7 92.9) (end 96.9 92.9) (width 0.25) (layer "B.Cu") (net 3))
 (segment (start 96.9 92.9) (end 97 93) (width 0.25) (layer "B.Cu") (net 3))
 (segment (start 97 93) (end 97.1 93) (width 0.25) (layer "B.Cu") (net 3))
 (segment (start 97.1 93) (end 97.2 93.1) (width 0.25) (layer "B.Cu") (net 3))
 (segment (start 97.2 93.1) (end 97.3 93.1) (width 0.25) (layer "B.Cu") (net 3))
 (segment (start 97.3 93.1) (end 97.4 93.2) (width 0.25) (layer "B.Cu") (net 3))
 (segment (start 97.4 93.2) (end 97.5 93.2) (width 0.25) (layer "B.Cu") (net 3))
 (segment (start 97.5 93.2) (end 97.6 93.3) (width 0.25) (layer "B.Cu") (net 3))
 (segment (start 97.6 93.3) (end 97.7 93.3) (width 0.25) (layer "B.Cu") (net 3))
 (segment (start 97.7 93.3) (end 97.8 93.4) (width 0.25) (layer "B.Cu") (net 3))
 (segment (start 97.8 93.4) (end 98 93.4) (width 0.25) (layer "B.Cu") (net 3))
 (segment (start 98 93.4) (end 98.1 93.5) (width 0.25) (layer "B.Cu") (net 3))
 (segment (start 98.1 93.5) (end 98.2 93.5) (width 0.25) (layer "B.Cu") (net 3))
 (segment (start 98.2 93.5) (end 98.3 93.6) (width 0.25) (layer "B.Cu") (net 3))
 (via (at 94.7 91.5) (size 1) (drill 0.55) (layers "F.Cu" "B.Cu") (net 3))
 (segment (start 91.5 93.8) (end 93.5 93.8) (width 0.25) (layer "B.Cu") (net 1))
 (segment (start 94.1 93) (end 94.1 92.3) (width 0.25) (layer "B.Cu") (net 1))
 (segment (start 94.1 92.3) (end 93.9 92.1) (width 0.25) (layer "B.Cu") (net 1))
 (segment (start 93.9 92.1) (end 93.9 92) (width 0.25) (layer "B.Cu") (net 1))
 (segment (start 93.9 92) (end 93.8 91.9) (width 0.25) (layer "B.Cu") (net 1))
 (segment (start 93.8 91.9) (end 93.8 91.1) (width 0.25) (layer "B.Cu") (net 1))
 (segment (start 93.8 91.1) (end 93.9 91) (width 0.25) (layer "B.Cu") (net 1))
 (segment (start 93.9 91) (end 93.9 90.9) (width 0.25) (layer "B.Cu") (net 1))
 (segment (start 93.9 90.9) (end 95.3 89.5) (width 0.25) (layer "B.Cu") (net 1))
 (segment (start 95.3 89.5) (end 95.6 89.2) (width 0.25) (layer "F.Cu") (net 1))
 (segment (start 95.6 89.2) (end 95.6 88.4) (width 0.25) (layer "F.Cu") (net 1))
 (segment (start 95.6 88.4) (end 95.7 88.3) (width 0.25) (layer "F.Cu") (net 1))
 (segment (start 95.7 88.3) (end 95.7 88.2) (width 0.25) (layer "F.Cu") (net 1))
 (segment (start 95.7 88.2) (end 96.3 87.6) (width 0.25) (layer "F.Cu") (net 1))
 (via (at 95.3 89.5) (size 1) (drill 0.55) (layers "F.Cu" "B.Cu") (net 1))
 (gr_line (start 93.323 85.8669) (end 98.442 85.8669) (stroke (width 0.1) (type default)) (layer "Edge.Cuts"))
 (gr_line (start 98.442 85.8669) (end 98.6646 87.9813) (stroke (width 0.1) (type default)) (layer "Edge.Cuts"))
 (gr_line (start 98.6646 87.9813) (end 100.2226 90.207) (stroke (width 0.1) (type default)) (layer "Edge.Cuts"))
 (gr_line (start 100.2226 90.207) (end 102.8934 91.5424) (stroke (width 0.1) (type default)) (layer "Edge.Cuts"))
 (gr_line (start 102.8934 91.5424) (end 105.5642 91.5424) (stroke (width 0.1) (type default)) (layer "Edge.Cuts"))
 (gr_line (start 105.5642 91.5424) (end 107.5673 90.0957) (stroke (width 0.1) (type default)) (layer "Edge.Cuts"))
 (gr_line (start 107.5673 90.0957) (end 108.6802 90.3183) (stroke (width 0.1) (type default)) (layer "Edge.Cuts"))
 (gr_line (start 108.6802 90.3183) (end 112.2412 97.1066) (stroke (width 0.1) (type default)) (layer "Edge.Cuts"))
 (gr_line (start 112.2412 97.1066) (end 114.2444 100.8903) (stroke (width 0.1) (type default)) (layer "Edge.Cuts"))
 (gr_line (start 114.2444 100.8903) (end 114.2444 106.677) (stroke (width 0.1) (type default)) (layer "Edge.Cuts"))
 (gr_line (start 114.2444 106.677) (end 111.5735 108.9027) (stroke (width 0.1) (type default)) (layer "Edge.Cuts"))
 (gr_line (start 111.5735 108.9027) (end 87.9813 108.9027) (stroke (width 0.1) (type default)) (layer "Edge.Cuts"))
 (gr_line (start 87.9813 108.9027) (end 85.6444 100.8903) (stroke (width 0.1) (type default)) (layer "Edge.Cuts"))
 (gr_line (start 85.6444 100.8903) (end 88.2039 94.8809) (stroke (width 0.1) (type default)) (layer "Edge.Cuts"))
 (gr_line (start 88.2039 94.8809) (end 93.323 85.8669) (stroke (width 0.1) (type default)) (layer "Edge.Cuts")))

